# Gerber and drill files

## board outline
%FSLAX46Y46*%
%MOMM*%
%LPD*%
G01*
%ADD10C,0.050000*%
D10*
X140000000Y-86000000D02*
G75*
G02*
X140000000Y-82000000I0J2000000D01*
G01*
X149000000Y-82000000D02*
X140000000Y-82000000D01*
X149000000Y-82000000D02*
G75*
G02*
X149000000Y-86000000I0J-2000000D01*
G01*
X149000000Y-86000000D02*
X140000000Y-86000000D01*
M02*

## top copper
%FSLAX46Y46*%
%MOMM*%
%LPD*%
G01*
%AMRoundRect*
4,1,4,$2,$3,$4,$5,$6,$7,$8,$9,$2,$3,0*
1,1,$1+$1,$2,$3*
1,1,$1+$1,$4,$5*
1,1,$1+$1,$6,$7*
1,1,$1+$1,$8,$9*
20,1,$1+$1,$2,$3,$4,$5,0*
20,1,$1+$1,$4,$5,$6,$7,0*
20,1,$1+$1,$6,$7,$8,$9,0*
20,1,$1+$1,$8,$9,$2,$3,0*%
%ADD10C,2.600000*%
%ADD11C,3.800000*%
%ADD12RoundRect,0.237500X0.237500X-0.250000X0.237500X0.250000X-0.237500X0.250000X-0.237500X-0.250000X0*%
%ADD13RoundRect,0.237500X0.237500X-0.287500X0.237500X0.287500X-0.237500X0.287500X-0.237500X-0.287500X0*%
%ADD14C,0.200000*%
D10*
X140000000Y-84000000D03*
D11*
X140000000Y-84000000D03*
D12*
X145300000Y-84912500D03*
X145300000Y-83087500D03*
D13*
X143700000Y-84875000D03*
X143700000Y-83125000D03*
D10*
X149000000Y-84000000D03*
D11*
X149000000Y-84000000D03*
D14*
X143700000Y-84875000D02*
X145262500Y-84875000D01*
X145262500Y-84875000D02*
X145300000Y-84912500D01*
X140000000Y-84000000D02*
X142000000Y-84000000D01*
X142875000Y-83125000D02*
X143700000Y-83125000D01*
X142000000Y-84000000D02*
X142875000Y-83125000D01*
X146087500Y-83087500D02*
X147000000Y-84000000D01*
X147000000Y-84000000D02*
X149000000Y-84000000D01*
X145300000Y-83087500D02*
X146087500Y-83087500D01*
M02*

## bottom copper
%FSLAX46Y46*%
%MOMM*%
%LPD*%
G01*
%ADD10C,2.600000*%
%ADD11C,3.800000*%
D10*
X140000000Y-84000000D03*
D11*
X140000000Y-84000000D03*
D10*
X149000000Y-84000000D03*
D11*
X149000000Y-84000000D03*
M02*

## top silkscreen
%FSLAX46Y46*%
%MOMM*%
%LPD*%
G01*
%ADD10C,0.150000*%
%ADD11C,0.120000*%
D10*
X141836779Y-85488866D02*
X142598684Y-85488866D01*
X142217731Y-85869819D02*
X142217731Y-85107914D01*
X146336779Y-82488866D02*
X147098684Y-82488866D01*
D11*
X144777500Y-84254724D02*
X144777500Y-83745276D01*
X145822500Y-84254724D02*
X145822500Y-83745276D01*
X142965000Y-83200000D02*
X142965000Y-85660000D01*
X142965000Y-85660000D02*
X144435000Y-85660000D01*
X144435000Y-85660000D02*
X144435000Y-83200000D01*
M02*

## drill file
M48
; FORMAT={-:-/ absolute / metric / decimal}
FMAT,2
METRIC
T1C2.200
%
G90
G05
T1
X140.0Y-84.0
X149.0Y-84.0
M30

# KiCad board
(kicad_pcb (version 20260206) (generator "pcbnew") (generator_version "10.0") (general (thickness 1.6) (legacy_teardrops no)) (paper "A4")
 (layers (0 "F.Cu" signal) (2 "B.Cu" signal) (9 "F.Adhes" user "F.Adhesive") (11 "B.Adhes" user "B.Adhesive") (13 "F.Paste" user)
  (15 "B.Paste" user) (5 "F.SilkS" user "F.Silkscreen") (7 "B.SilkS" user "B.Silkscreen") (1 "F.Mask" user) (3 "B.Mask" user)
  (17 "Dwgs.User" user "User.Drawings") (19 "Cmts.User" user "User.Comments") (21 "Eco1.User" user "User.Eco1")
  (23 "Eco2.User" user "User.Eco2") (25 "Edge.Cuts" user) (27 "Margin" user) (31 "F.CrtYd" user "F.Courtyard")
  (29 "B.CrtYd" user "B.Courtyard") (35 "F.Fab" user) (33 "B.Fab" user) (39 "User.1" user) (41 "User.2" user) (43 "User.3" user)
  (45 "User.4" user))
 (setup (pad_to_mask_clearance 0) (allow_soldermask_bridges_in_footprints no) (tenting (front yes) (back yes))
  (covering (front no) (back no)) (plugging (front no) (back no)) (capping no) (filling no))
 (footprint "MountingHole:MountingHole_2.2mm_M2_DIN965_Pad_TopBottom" (layer "F.Cu") (at 140 84)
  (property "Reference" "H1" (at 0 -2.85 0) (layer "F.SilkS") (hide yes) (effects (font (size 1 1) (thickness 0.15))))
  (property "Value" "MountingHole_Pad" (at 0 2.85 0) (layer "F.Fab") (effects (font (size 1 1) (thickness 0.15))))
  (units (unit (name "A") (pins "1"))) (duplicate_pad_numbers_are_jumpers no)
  (pad "1" thru_hole circle (at 0 0) (size 2.6 2.6) (drill 2.2) (layers "*.Cu" "*.Mask") (remove_unused_layers no) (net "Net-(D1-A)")
   (zone_connect 2))
  (pad "1" connect circle (at 0 0) (size 3.8 3.8) (layers "F.Cu" "F.Mask") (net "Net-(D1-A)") (zone_connect 2))
  (pad "1" connect circle (at 0 0) (size 3.8 3.8) (layers "B.Cu" "B.Mask") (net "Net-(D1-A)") (zone_connect 2)))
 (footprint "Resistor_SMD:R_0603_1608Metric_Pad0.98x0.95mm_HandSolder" (layer "F.Cu") (at 145.3 84 90)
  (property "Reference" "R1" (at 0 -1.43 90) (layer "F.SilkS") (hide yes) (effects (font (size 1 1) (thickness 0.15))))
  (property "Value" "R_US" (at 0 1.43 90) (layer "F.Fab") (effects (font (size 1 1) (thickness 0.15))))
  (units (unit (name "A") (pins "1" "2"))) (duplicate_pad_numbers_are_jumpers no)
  (fp_line (start -0.254724 -0.5225) (end 0.254724 -0.5225) (stroke (width 0.12) (type solid)) (layer "F.SilkS"))
  (fp_line (start -0.254724 0.5225) (end 0.254724 0.5225) (stroke (width 0.12) (type solid)) (layer "F.SilkS"))
  (pad "1" smd roundrect (at -0.9125 0 90) (size 0.975 0.95) (layers "F.Cu" "F.Mask" "F.Paste") (roundrect_rratio 0.25) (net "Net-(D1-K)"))
  (pad "2" smd roundrect (at 0.9125 0 90) (size 0.975 0.95) (layers "F.Cu" "F.Mask" "F.Paste") (roundrect_rratio 0.25) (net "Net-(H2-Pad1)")))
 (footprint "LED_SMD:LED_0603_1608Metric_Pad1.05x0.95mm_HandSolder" (layer "F.Cu") (at 143.7 84 90)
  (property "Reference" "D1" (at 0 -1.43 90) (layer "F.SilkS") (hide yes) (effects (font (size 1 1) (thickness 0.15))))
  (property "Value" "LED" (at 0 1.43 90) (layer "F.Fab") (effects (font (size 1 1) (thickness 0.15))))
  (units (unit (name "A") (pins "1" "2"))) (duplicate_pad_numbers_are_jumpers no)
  (fp_line (start 0.8 -0.735) (end -1.66 -0.735) (stroke (width 0.12) (type solid)) (layer "F.SilkS"))
  (fp_line (start -1.66 -0.735) (end -1.66 0.735) (stroke (width 0.12) (type solid)) (layer "F.SilkS"))
  (fp_line (start -1.66 0.735) (end 0.8 0.735) (stroke (width 0.12) (type solid)) (layer "F.SilkS"))
  (pad "1" smd roundrect (at -0.875 0 90) (size 1.05 0.95) (layers "F.Cu" "F.Mask" "F.Paste") (roundrect_rratio 0.25) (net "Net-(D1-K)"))
  (pad "2" smd roundrect (at 0.875 0 90) (size 1.05 0.95) (layers "F.Cu" "F.Mask" "F.Paste") (roundrect_rratio 0.25) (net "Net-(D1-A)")))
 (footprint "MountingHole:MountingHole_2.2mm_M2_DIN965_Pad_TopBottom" (layer "F.Cu") (at 149 84)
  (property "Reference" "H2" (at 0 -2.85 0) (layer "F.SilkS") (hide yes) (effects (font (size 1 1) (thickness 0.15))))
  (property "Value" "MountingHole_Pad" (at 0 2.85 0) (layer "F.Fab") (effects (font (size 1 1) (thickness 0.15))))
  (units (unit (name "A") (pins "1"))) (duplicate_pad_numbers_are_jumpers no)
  (pad "1" thru_hole circle (at 0 0) (size 2.6 2.6) (drill 2.2) (layers "*.Cu" "*.Mask") (remove_unused_layers no) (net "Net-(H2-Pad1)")
   (zone_connect 2))
  (pad "1" connect circle (at 0 0) (size 3.8 3.8) (layers "F.Cu" "F.Mask") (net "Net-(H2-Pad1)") (zone_connect 2))
  (pad "1" connect circle (at 0 0) (size 3.8 3.8) (layers "B.Cu" "B.Mask") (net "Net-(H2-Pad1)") (zone_connect 2)))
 (gr_arc (start 140 86) (mid 138 84) (end 140 82) (stroke (width 0.05) (type default)) (layer "Edge.Cuts"))
 (gr_line (start 149 82) (end 140 82) (stroke (width 0.05) (type default)) (layer "Edge.Cuts"))
 (gr_arc (start 149 82) (mid 151 84) (end 149 86) (stroke (width 0.05) (type default)) (layer "Edge.Cuts"))
 (gr_line (start 149 86) (end 140 86) (stroke (width 0.05) (type default)) (layer "Edge.Cuts"))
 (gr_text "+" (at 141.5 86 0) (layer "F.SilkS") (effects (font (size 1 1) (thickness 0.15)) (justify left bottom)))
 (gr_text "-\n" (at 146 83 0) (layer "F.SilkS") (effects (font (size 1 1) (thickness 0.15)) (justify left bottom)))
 (segment (start 143.7 84.875) (end 145.2625 84.875) (width 0.2) (layer "F.Cu") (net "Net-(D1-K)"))
 (segment (start 145.2625 84.875) (end 145.3 84.9125) (width 0.2) (layer "F.Cu") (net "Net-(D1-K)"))
 (segment (start 140 84) (end 142 84) (width 0.2) (layer "F.Cu") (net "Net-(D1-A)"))
 (segment (start 142.875 83.125) (end 143.7 83.125) (width 0.2) (layer "F.Cu") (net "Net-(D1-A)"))
 (segment (start 142 84) (end 142.875 83.125) (width 0.2) (layer "F.Cu") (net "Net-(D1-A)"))
 (segment (start 146.0875 83.0875) (end 147 84) (width 0.2) (layer "F.Cu") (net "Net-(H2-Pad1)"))
 (segment (start 147 84) (end 149 84) (width 0.2) (layer "F.Cu") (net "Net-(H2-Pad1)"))
 (segment (start 145.3 83.0875) (end 146.0875 83.0875) (width 0.2) (layer "F.Cu") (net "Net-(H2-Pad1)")))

